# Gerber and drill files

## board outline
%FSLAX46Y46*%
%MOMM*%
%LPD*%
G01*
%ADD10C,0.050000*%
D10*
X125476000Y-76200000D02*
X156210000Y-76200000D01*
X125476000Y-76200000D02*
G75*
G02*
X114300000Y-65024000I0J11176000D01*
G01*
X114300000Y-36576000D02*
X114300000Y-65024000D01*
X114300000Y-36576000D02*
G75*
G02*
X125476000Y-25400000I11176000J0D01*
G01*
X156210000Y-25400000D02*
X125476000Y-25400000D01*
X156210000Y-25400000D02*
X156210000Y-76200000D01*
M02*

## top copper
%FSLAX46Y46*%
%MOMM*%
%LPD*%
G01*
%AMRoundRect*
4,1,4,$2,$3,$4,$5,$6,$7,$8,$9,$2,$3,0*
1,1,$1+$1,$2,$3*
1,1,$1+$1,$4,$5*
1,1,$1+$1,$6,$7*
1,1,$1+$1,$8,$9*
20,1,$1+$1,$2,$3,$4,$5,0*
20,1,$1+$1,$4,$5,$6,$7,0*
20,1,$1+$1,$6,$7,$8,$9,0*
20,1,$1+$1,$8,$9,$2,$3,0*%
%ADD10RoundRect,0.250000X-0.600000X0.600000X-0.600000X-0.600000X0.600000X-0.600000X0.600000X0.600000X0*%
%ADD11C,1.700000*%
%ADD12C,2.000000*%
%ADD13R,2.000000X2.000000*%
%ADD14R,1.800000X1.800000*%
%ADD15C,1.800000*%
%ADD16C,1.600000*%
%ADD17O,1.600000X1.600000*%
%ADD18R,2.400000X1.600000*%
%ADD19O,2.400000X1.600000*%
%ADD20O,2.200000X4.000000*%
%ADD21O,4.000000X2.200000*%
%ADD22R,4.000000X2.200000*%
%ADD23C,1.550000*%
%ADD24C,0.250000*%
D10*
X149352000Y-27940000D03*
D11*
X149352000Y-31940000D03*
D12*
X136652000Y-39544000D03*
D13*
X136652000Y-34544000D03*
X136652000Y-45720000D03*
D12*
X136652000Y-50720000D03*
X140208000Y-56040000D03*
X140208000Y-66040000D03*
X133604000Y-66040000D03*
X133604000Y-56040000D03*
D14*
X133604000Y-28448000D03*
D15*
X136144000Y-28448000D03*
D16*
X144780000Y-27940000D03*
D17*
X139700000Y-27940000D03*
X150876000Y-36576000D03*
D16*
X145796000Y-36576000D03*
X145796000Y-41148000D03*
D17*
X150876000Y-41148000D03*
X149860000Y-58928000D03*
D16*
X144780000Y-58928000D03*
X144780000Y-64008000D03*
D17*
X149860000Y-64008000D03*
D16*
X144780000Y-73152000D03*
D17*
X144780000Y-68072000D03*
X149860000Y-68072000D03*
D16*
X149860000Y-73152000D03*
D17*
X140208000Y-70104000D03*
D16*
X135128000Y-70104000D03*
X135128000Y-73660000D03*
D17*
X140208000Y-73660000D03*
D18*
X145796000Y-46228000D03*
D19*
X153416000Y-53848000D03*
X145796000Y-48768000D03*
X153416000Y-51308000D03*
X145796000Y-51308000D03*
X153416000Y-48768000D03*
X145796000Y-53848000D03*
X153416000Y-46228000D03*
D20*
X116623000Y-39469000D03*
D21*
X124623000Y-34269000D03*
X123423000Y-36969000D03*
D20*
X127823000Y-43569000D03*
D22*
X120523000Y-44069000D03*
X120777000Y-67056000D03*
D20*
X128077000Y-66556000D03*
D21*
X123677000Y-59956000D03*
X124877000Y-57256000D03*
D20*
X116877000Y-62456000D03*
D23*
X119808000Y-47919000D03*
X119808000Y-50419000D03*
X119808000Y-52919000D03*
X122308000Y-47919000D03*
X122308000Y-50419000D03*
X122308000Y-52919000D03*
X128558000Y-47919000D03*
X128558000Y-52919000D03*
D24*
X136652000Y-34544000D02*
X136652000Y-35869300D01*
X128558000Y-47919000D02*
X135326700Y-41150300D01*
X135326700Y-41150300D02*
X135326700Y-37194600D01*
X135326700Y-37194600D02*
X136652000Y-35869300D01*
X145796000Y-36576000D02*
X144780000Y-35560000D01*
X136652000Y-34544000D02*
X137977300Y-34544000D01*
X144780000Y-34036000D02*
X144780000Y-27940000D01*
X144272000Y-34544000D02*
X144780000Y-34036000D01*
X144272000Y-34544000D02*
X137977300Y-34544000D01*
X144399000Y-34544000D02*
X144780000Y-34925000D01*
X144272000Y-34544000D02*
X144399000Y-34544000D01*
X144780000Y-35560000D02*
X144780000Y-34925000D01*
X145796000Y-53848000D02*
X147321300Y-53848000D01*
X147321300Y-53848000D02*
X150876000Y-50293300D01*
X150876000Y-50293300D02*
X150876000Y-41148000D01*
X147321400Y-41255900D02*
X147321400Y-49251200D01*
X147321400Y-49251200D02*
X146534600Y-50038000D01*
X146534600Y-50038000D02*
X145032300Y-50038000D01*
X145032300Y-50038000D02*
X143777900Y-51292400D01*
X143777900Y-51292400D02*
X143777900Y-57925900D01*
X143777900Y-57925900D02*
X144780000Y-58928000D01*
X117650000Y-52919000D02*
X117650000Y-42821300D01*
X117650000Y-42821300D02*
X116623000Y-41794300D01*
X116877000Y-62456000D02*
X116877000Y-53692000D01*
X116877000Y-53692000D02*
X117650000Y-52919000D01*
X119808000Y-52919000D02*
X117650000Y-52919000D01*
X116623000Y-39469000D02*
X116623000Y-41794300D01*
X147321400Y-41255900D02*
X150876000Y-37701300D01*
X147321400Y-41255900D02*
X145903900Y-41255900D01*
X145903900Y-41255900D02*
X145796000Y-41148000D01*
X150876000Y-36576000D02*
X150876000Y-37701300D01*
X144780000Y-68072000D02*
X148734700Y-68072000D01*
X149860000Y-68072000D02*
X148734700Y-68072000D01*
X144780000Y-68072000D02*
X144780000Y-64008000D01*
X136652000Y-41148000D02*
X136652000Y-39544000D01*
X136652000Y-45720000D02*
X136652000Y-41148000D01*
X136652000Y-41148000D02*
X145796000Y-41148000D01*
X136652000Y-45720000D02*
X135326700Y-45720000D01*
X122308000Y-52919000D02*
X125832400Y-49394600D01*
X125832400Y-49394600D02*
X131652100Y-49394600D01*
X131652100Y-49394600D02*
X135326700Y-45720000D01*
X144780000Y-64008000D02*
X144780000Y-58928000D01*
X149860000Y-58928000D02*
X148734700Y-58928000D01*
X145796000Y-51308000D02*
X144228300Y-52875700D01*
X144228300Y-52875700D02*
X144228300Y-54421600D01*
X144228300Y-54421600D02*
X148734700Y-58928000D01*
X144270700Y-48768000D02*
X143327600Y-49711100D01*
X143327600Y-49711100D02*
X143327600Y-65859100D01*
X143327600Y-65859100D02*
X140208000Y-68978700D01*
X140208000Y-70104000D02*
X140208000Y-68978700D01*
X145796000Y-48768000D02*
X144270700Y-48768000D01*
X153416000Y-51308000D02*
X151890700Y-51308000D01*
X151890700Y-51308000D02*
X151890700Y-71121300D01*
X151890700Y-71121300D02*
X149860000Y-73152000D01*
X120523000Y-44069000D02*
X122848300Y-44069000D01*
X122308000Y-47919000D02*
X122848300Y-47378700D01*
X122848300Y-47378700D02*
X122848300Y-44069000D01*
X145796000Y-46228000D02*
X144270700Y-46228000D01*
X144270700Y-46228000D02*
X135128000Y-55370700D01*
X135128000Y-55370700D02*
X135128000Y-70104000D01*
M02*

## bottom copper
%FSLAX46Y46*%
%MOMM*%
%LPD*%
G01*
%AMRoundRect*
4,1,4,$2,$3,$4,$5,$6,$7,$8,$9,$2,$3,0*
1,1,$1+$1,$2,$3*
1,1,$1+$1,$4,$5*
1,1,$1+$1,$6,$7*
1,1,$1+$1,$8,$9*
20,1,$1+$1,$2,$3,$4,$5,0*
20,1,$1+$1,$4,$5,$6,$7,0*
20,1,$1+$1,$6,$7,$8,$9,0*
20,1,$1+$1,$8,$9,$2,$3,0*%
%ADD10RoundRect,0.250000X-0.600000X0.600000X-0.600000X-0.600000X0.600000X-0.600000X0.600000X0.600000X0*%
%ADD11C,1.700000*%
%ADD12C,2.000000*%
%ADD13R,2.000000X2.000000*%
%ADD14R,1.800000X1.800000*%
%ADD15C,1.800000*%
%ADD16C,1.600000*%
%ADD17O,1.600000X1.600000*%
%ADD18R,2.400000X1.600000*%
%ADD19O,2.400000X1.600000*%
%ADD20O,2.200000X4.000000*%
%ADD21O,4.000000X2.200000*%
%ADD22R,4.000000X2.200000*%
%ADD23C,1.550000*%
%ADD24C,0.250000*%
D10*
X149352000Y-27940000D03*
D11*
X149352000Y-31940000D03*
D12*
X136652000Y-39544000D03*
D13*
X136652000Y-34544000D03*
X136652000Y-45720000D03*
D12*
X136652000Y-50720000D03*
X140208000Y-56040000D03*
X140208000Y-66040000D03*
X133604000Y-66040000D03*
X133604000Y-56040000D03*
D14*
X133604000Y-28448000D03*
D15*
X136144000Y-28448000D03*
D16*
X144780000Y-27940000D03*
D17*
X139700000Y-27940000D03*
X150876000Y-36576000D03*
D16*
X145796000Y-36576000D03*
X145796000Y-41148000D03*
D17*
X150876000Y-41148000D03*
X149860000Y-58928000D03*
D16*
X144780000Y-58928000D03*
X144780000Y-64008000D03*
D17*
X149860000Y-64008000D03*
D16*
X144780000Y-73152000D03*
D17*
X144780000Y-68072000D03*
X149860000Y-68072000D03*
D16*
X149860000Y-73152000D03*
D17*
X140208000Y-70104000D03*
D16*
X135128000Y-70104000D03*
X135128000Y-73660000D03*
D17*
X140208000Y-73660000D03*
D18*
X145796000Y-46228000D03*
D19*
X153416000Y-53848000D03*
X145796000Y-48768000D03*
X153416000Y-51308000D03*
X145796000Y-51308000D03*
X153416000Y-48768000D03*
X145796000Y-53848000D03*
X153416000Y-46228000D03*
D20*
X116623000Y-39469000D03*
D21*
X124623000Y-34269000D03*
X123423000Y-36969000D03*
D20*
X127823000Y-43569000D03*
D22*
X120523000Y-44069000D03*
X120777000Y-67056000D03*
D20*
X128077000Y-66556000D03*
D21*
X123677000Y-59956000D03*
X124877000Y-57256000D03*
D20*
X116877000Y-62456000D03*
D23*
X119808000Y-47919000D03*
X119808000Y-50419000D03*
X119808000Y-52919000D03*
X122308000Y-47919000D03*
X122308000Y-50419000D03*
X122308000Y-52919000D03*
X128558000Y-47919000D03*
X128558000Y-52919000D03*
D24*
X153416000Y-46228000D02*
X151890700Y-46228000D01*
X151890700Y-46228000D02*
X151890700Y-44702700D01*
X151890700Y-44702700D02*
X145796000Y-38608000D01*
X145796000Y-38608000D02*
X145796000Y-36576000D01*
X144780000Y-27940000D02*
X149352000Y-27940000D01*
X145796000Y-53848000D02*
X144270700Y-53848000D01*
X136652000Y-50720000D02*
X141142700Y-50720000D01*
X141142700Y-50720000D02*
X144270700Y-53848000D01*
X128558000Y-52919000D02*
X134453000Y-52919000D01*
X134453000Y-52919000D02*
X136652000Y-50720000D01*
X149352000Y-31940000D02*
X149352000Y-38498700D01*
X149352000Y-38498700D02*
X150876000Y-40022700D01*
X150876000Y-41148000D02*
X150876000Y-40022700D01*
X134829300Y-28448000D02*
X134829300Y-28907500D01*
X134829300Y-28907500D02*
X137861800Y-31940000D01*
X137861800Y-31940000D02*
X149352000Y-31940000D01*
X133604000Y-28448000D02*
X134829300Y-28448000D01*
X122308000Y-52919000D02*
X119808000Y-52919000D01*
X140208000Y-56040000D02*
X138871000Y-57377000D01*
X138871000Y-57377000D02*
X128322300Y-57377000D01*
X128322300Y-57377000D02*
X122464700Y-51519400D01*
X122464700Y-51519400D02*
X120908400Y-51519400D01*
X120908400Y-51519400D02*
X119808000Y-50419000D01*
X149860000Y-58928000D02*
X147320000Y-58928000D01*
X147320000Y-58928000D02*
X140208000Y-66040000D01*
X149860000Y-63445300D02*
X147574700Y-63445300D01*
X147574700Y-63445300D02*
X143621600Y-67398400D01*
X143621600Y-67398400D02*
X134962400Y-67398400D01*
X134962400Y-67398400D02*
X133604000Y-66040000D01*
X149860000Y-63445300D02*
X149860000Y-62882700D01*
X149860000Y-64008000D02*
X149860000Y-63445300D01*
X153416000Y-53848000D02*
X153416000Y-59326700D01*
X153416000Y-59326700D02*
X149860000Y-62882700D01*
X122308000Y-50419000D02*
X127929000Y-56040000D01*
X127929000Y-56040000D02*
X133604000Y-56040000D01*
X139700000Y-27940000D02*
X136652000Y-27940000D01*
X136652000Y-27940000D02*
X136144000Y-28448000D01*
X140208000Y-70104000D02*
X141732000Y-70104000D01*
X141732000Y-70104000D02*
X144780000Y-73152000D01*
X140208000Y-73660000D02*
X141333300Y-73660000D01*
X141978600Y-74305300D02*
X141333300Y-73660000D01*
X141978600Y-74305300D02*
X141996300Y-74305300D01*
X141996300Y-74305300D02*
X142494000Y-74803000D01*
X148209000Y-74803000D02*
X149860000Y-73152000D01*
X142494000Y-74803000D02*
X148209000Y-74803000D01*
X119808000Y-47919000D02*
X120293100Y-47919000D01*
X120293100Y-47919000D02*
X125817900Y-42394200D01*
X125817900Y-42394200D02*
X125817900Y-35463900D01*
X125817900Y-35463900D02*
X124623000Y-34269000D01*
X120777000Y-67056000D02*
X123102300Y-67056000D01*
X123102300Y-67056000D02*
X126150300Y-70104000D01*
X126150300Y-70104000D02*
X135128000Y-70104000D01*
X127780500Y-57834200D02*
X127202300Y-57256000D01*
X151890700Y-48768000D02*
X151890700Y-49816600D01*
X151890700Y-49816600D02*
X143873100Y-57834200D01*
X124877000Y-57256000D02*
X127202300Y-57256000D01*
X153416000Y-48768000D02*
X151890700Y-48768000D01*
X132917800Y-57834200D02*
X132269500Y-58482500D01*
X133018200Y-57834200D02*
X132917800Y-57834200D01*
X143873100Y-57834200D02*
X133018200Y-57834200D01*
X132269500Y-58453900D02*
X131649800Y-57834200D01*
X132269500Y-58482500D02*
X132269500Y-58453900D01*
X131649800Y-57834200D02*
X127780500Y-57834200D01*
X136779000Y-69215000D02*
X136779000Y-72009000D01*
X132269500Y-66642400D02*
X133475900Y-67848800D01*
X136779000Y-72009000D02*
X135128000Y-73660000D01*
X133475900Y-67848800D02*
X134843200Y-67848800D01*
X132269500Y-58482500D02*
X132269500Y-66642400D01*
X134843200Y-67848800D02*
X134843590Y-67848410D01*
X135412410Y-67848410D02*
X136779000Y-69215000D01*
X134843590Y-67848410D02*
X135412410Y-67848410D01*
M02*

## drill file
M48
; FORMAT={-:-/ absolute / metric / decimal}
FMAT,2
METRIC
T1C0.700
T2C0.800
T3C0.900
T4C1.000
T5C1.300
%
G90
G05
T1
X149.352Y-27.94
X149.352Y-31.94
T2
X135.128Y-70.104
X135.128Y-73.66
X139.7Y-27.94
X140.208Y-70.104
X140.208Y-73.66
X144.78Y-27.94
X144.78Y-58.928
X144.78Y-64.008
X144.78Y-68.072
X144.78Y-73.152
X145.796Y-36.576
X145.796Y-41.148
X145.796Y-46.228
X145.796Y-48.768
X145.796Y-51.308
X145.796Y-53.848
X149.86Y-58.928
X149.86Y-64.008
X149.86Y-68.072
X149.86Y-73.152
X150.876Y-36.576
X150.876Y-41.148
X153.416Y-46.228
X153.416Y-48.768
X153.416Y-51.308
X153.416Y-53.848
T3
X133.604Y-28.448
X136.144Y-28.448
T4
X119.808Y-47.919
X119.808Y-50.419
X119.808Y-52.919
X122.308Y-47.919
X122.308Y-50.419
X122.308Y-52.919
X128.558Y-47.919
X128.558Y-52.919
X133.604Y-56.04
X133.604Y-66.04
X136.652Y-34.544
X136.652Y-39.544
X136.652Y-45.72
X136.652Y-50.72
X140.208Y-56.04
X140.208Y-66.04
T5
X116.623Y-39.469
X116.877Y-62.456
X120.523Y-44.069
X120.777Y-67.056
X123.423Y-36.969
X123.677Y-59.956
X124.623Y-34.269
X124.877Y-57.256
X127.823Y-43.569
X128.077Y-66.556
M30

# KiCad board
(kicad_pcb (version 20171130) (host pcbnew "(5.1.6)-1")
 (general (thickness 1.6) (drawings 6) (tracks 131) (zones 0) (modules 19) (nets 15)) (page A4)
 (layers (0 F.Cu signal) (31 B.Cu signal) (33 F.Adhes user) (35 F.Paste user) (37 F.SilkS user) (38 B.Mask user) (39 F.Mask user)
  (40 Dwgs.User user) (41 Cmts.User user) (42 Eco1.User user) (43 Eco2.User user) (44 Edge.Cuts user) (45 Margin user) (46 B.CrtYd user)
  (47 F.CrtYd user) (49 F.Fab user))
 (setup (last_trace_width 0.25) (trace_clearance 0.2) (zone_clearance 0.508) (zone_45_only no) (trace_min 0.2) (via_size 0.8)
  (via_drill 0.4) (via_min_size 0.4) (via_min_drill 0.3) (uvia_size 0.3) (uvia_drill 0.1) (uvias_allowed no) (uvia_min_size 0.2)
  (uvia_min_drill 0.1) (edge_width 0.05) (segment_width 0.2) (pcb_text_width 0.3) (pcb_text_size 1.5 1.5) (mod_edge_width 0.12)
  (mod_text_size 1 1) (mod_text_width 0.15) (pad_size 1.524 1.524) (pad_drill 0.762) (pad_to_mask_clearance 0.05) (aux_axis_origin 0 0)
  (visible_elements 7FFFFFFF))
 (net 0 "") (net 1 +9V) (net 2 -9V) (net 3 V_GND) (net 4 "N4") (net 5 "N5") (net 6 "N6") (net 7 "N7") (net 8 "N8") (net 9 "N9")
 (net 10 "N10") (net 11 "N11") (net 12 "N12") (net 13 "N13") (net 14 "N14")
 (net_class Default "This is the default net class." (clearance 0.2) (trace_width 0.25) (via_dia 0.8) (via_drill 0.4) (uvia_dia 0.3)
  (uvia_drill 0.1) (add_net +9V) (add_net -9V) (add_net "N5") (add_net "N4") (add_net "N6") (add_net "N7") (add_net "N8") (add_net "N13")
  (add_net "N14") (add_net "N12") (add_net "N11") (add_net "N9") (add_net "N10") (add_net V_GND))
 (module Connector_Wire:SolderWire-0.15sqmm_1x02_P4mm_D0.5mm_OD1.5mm (layer F.Cu) (at 149.352 27.94 270)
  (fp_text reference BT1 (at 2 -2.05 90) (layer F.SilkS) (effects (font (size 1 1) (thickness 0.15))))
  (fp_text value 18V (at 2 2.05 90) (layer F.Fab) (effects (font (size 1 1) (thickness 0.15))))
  (pad 1 thru_hole roundrect (at 0 0 270) (size 1.7 1.7) (drill 0.7) (layers *.Cu *.Mask) (roundrect_rratio 0.147059) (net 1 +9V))
  (pad 2 thru_hole circle (at 4 0 270) (size 1.7 1.7) (drill 0.7) (layers *.Cu *.Mask) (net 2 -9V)))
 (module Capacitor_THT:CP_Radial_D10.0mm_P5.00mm (layer F.Cu) (at 136.652 34.544 270)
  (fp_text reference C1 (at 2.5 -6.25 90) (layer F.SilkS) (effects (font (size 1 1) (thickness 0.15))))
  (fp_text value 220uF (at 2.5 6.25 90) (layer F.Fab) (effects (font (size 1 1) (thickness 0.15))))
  (pad 2 thru_hole circle (at 5 0 270) (size 2 2) (drill 1) (layers *.Cu *.Mask) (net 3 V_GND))
  (pad 1 thru_hole rect (at 0 0 270) (size 2 2) (drill 1) (layers *.Cu *.Mask) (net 1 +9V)))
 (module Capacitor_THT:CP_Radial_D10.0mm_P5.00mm (layer F.Cu) (at 136.652 45.72 270)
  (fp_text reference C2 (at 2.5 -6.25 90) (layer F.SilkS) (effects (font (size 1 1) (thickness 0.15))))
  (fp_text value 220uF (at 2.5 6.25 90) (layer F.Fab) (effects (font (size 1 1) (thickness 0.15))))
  (pad 1 thru_hole rect (at 0 0 270) (size 2 2) (drill 1) (layers *.Cu *.Mask) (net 3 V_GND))
  (pad 2 thru_hole circle (at 5 0 270) (size 2 2) (drill 1) (layers *.Cu *.Mask) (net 2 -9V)))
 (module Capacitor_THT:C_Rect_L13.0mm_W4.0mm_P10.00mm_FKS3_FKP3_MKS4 (layer F.Cu) (at 140.208 66.04 90)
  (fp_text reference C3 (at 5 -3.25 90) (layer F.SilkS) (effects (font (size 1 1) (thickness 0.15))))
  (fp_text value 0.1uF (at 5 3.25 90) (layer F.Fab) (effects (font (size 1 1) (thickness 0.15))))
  (pad 2 thru_hole circle (at 10 0 90) (size 2 2) (drill 1) (layers *.Cu *.Mask) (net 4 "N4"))
  (pad 1 thru_hole circle (at 0 0 90) (size 2 2) (drill 1) (layers *.Cu *.Mask) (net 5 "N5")))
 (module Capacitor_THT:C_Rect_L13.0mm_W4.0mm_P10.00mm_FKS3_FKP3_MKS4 (layer F.Cu) (at 133.604 66.04 90)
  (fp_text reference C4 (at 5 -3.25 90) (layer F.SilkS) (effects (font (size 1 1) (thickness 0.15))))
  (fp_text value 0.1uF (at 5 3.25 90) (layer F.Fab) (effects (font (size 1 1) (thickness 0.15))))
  (pad 1 thru_hole circle (at 0 0 90) (size 2 2) (drill 1) (layers *.Cu *.Mask) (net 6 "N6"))
  (pad 2 thru_hole circle (at 10 0 90) (size 2 2) (drill 1) (layers *.Cu *.Mask) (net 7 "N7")))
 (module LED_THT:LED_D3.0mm (layer F.Cu) (at 133.604 28.448)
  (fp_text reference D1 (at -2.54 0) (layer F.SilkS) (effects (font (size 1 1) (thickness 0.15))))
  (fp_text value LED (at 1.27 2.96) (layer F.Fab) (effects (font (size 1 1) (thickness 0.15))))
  (pad 1 thru_hole rect (at 0 0) (size 1.8 1.8) (drill 0.9) (layers *.Cu *.Mask) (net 2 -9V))
  (pad 2 thru_hole circle (at 2.54 0) (size 1.8 1.8) (drill 0.9) (layers *.Cu *.Mask) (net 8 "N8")))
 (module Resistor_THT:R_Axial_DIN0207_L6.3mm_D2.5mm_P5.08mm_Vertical (layer F.Cu) (at 144.78 27.94 180)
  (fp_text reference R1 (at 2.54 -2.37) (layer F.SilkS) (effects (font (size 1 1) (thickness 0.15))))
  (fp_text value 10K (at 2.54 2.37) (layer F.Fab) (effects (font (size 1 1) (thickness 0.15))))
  (pad 1 thru_hole circle (at 0 0 180) (size 1.6 1.6) (drill 0.8) (layers *.Cu *.Mask) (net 1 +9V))
  (pad 2 thru_hole oval (at 5.08 0 180) (size 1.6 1.6) (drill 0.8) (layers *.Cu *.Mask) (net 8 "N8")))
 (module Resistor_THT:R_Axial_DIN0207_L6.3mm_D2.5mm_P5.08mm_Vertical (layer F.Cu) (at 145.796 36.576)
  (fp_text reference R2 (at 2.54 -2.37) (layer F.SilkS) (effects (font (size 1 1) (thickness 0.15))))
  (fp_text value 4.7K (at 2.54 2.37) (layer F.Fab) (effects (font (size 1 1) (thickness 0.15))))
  (pad 2 thru_hole oval (at 5.08 0) (size 1.6 1.6) (drill 0.8) (layers *.Cu *.Mask) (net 3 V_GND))
  (pad 1 thru_hole circle (at 0 0) (size 1.6 1.6) (drill 0.8) (layers *.Cu *.Mask) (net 1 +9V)))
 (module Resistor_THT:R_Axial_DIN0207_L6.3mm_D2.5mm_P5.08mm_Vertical (layer F.Cu) (at 145.796 41.148)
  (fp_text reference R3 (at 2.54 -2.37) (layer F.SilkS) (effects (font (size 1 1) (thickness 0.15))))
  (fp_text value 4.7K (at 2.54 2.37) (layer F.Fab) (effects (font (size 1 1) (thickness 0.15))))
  (pad 1 thru_hole circle (at 0 0) (size 1.6 1.6) (drill 0.8) (layers *.Cu *.Mask) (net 3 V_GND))
  (pad 2 thru_hole oval (at 5.08 0) (size 1.6 1.6) (drill 0.8) (layers *.Cu *.Mask) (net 2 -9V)))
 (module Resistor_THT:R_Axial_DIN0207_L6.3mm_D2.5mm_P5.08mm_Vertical (layer F.Cu) (at 144.78 58.928)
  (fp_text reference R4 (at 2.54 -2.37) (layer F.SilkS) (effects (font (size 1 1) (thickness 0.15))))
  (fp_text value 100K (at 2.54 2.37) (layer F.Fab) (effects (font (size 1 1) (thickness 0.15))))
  (pad 2 thru_hole oval (at 5.08 0) (size 1.6 1.6) (drill 0.8) (layers *.Cu *.Mask) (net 5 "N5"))
  (pad 1 thru_hole circle (at 0 0) (size 1.6 1.6) (drill 0.8) (layers *.Cu *.Mask) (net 3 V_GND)))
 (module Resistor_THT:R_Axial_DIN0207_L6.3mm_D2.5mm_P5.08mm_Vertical (layer F.Cu) (at 144.78 64.008)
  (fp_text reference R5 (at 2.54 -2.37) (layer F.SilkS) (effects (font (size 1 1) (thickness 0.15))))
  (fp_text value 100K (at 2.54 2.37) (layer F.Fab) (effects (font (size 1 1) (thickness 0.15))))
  (pad 1 thru_hole circle (at 0 0) (size 1.6 1.6) (drill 0.8) (layers *.Cu *.Mask) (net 3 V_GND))
  (pad 2 thru_hole oval (at 5.08 0) (size 1.6 1.6) (drill 0.8) (layers *.Cu *.Mask) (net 6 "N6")))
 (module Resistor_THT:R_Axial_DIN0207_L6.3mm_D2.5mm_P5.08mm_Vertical (layer F.Cu) (at 144.78 73.152 90)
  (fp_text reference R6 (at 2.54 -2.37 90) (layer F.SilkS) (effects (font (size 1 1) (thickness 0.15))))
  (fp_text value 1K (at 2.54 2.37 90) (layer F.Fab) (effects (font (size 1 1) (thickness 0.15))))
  (pad 1 thru_hole circle (at 0 0 90) (size 1.6 1.6) (drill 0.8) (layers *.Cu *.Mask) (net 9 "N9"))
  (pad 2 thru_hole oval (at 5.08 0 90) (size 1.6 1.6) (drill 0.8) (layers *.Cu *.Mask) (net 3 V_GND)))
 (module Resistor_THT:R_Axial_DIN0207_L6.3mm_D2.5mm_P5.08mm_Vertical (layer F.Cu) (at 149.86 73.152 90)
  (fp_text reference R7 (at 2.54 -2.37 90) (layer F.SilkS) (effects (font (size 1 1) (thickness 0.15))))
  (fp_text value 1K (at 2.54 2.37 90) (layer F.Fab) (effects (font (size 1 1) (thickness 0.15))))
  (pad 2 thru_hole oval (at 5.08 0 90) (size 1.6 1.6) (drill 0.8) (layers *.Cu *.Mask) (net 3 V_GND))
  (pad 1 thru_hole circle (at 0 0 90) (size 1.6 1.6) (drill 0.8) (layers *.Cu *.Mask) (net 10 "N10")))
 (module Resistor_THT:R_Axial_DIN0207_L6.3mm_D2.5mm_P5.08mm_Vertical (layer F.Cu) (at 135.128 70.104)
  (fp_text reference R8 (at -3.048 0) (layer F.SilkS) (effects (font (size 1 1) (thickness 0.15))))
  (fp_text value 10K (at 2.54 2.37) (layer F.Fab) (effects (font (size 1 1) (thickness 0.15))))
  (pad 2 thru_hole oval (at 5.08 0) (size 1.6 1.6) (drill 0.8) (layers *.Cu *.Mask) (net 9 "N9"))
  (pad 1 thru_hole circle (at 0 0) (size 1.6 1.6) (drill 0.8) (layers *.Cu *.Mask) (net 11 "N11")))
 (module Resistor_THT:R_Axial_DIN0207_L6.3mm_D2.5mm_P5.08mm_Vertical (layer F.Cu) (at 135.128 73.66)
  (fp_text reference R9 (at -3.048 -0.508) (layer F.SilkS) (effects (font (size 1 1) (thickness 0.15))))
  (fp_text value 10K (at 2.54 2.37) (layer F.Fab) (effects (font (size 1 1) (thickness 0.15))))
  (pad 1 thru_hole circle (at 0 0) (size 1.6 1.6) (drill 0.8) (layers *.Cu *.Mask) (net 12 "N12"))
  (pad 2 thru_hole oval (at 5.08 0) (size 1.6 1.6) (drill 0.8) (layers *.Cu *.Mask) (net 10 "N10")))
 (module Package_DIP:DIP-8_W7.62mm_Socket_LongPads (layer F.Cu) (at 145.796 46.228)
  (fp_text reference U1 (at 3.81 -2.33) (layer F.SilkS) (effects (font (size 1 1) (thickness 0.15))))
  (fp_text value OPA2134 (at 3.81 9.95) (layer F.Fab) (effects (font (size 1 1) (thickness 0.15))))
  (pad 1 thru_hole rect (at 0 0) (size 2.4 1.6) (drill 0.8) (layers *.Cu *.Mask) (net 11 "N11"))
  (pad 5 thru_hole oval (at 7.62 7.62) (size 2.4 1.6) (drill 0.8) (layers *.Cu *.Mask) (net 6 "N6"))
  (pad 2 thru_hole oval (at 0 2.54) (size 2.4 1.6) (drill 0.8) (layers *.Cu *.Mask) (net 9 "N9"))
  (pad 6 thru_hole oval (at 7.62 5.08) (size 2.4 1.6) (drill 0.8) (layers *.Cu *.Mask) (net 10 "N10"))
  (pad 3 thru_hole oval (at 0 5.08) (size 2.4 1.6) (drill 0.8) (layers *.Cu *.Mask) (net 5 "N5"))
  (pad 7 thru_hole oval (at 7.62 2.54) (size 2.4 1.6) (drill 0.8) (layers *.Cu *.Mask) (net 12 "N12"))
  (pad 4 thru_hole oval (at 0 7.62) (size 2.4 1.6) (drill 0.8) (layers *.Cu *.Mask) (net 2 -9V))
  (pad 8 thru_hole oval (at 7.62 0) (size 2.4 1.6) (drill 0.8) (layers *.Cu *.Mask) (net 1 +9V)))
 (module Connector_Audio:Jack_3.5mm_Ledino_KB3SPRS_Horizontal (layer F.Cu) (at 120.523 44.069)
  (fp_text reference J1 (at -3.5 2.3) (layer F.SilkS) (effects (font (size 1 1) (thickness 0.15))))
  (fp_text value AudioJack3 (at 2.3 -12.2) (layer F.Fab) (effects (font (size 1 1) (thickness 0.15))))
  (pad S thru_hole oval (at -3.9 -4.6) (size 2.2 4) (drill 1.3) (layers *.Cu *.Mask) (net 3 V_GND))
  (pad R thru_hole oval (at 4.1 -9.8) (size 4 2.2) (drill 1.3) (layers *.Cu *.Mask) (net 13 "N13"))
  (pad RN thru_hole oval (at 2.9 -7.1) (size 4 2.2) (drill 1.3) (layers *.Cu *.Mask))
  (pad TN thru_hole oval (at 7.3 -0.5 90) (size 4 2.2) (drill 1.3) (layers *.Cu *.Mask))
  (pad T thru_hole rect (at 0 0) (size 4 2.2) (drill 1.3) (layers *.Cu *.Mask) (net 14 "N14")))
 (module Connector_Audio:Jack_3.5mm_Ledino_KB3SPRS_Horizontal (layer F.Cu) (at 120.777 67.056)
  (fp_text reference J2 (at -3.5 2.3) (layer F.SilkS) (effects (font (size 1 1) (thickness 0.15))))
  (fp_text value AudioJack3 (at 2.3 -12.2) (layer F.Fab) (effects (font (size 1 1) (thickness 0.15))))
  (pad T thru_hole rect (at 0 0) (size 4 2.2) (drill 1.3) (layers *.Cu *.Mask) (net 11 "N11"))
  (pad TN thru_hole oval (at 7.3 -0.5 90) (size 4 2.2) (drill 1.3) (layers *.Cu *.Mask))
  (pad RN thru_hole oval (at 2.9 -7.1) (size 4 2.2) (drill 1.3) (layers *.Cu *.Mask))
  (pad R thru_hole oval (at 4.1 -9.8) (size 4 2.2) (drill 1.3) (layers *.Cu *.Mask) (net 12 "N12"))
  (pad S thru_hole oval (at -3.9 -4.6) (size 2.2 4) (drill 1.3) (layers *.Cu *.Mask) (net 3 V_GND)))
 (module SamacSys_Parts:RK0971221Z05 (layer F.Cu) (at 114.808 50.419 180)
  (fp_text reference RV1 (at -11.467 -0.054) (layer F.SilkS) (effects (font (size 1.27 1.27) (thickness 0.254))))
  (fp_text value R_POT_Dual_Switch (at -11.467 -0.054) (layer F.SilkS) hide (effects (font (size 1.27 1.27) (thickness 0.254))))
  (pad 1 thru_hole circle (at -5 2.5 180) (size 1.55 1.55) (drill 1) (layers *.Cu *.Mask) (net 13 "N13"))
  (pad 2 thru_hole circle (at -5 0 180) (size 1.55 1.55) (drill 1) (layers *.Cu *.Mask) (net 4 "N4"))
  (pad 3 thru_hole circle (at -5 -2.5 180) (size 1.55 1.55) (drill 1) (layers *.Cu *.Mask) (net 3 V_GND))
  (pad 4 thru_hole circle (at -7.5 2.5 180) (size 1.55 1.55) (drill 1) (layers *.Cu *.Mask) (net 14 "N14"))
  (pad 5 thru_hole circle (at -7.5 0 180) (size 1.55 1.55) (drill 1) (layers *.Cu *.Mask) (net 7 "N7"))
  (pad 6 thru_hole circle (at -7.5 -2.5 180) (size 1.55 1.55) (drill 1) (layers *.Cu *.Mask) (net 3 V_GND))
  (pad 7 thru_hole circle (at -13.75 2.5 180) (size 1.55 1.55) (drill 1) (layers *.Cu *.Mask) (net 1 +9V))
  (pad 8 thru_hole circle (at -13.75 -2.5 180) (size 1.55 1.55) (drill 1) (layers *.Cu *.Mask) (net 2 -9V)))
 (gr_line (start 125.476 76.2) (end 156.21 76.2) (layer Edge.Cuts) (width 0.05))
 (gr_arc (start 125.476 65.024) (end 114.3 65.024) (angle -90) (layer Edge.Cuts) (width 0.05))
 (gr_line (start 114.3 36.576) (end 114.3 65.024) (layer Edge.Cuts) (width 0.05))
 (gr_arc (start 125.476 36.576) (end 125.476 25.4) (angle -90) (layer Edge.Cuts) (width 0.05))
 (gr_line (start 156.21 25.4) (end 125.476 25.4) (layer Edge.Cuts) (width 0.05))
 (gr_line (start 156.21 25.4) (end 156.21 76.2) (layer Edge.Cuts) (width 0.05))
 (segment (start 153.416 46.228) (end 151.8907 46.228) (width 0.25) (layer B.Cu) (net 1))
 (segment (start 151.8907 46.228) (end 151.8907 44.7027) (width 0.25) (layer B.Cu) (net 1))
 (segment (start 151.8907 44.7027) (end 145.796 38.608) (width 0.25) (layer B.Cu) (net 1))
 (segment (start 145.796 38.608) (end 145.796 36.576) (width 0.25) (layer B.Cu) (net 1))
 (segment (start 136.652 34.544) (end 136.652 35.8693) (width 0.25) (layer F.Cu) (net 1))
 (segment (start 128.558 47.919) (end 135.3267 41.1503) (width 0.25) (layer F.Cu) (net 1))
 (segment (start 135.3267 41.1503) (end 135.3267 37.1946) (width 0.25) (layer F.Cu) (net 1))
 (segment (start 135.3267 37.1946) (end 136.652 35.8693) (width 0.25) (layer F.Cu) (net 1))
 (segment (start 145.796 36.576) (end 144.78 35.56) (width 0.25) (layer F.Cu) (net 1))
 (segment (start 136.652 34.544) (end 137.9773 34.544) (width 0.25) (layer F.Cu) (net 1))
 (segment (start 144.78 27.94) (end 149.352 27.94) (width 0.25) (layer B.Cu) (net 1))
 (segment (start 144.78 34.036) (end 144.78 27.94) (width 0.25) (layer F.Cu) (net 1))
 (segment (start 144.272 34.544) (end 144.78 34.036) (width 0.25) (layer F.Cu) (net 1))
 (segment (start 144.272 34.544) (end 137.9773 34.544) (width 0.25) (layer F.Cu) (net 1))
 (segment (start 144.399 34.544) (end 144.78 34.925) (width 0.25) (layer F.Cu) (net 1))
 (segment (start 144.272 34.544) (end 144.399 34.544) (width 0.25) (layer F.Cu) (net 1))
 (segment (start 144.78 35.56) (end 144.78 34.925) (width 0.25) (layer F.Cu) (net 1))
 (segment (start 145.796 53.848) (end 147.3213 53.848) (width 0.25) (layer F.Cu) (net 2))
 (segment (start 147.3213 53.848) (end 150.876 50.2933) (width 0.25) (layer F.Cu) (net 2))
 (segment (start 150.876 50.2933) (end 150.876 41.148) (width 0.25) (layer F.Cu) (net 2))
 (segment (start 145.796 53.848) (end 144.2707 53.848) (width 0.25) (layer B.Cu) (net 2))
 (segment (start 136.652 50.72) (end 141.1427 50.72) (width 0.25) (layer B.Cu) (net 2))
 (segment (start 141.1427 50.72) (end 144.2707 53.848) (width 0.25) (layer B.Cu) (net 2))
 (segment (start 128.558 52.919) (end 134.453 52.919) (width 0.25) (layer B.Cu) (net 2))
 (segment (start 134.453 52.919) (end 136.652 50.72) (width 0.25) (layer B.Cu) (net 2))
 (segment (start 149.352 31.94) (end 149.352 38.4987) (width 0.25) (layer B.Cu) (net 2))
 (segment (start 149.352 38.4987) (end 150.876 40.0227) (width 0.25) (layer B.Cu) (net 2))
 (segment (start 150.876 41.148) (end 150.876 40.0227) (width 0.25) (layer B.Cu) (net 2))
 (segment (start 134.8293 28.448) (end 134.8293 28.9075) (width 0.25) (layer B.Cu) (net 2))
 (segment (start 134.8293 28.9075) (end 137.8618 31.94) (width 0.25) (layer B.Cu) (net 2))
 (segment (start 137.8618 31.94) (end 149.352 31.94) (width 0.25) (layer B.Cu) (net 2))
 (segment (start 133.604 28.448) (end 134.8293 28.448) (width 0.25) (layer B.Cu) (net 2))
 (segment (start 147.3214 41.2559) (end 147.3214 49.2512) (width 0.25) (layer F.Cu) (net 3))
 (segment (start 147.3214 49.2512) (end 146.5346 50.038) (width 0.25) (layer F.Cu) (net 3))
 (segment (start 146.5346 50.038) (end 145.0323 50.038) (width 0.25) (layer F.Cu) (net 3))
 (segment (start 145.0323 50.038) (end 143.7779 51.2924) (width 0.25) (layer F.Cu) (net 3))
 (segment (start 143.7779 51.2924) (end 143.7779 57.9259) (width 0.25) (layer F.Cu) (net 3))
 (segment (start 143.7779 57.9259) (end 144.78 58.928) (width 0.25) (layer F.Cu) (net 3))
 (segment (start 117.65 52.919) (end 117.65 42.8213) (width 0.25) (layer F.Cu) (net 3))
 (segment (start 117.65 42.8213) (end 116.623 41.7943) (width 0.25) (layer F.Cu) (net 3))
 (segment (start 116.877 62.456) (end 116.877 53.692) (width 0.25) (layer F.Cu) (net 3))
 (segment (start 116.877 53.692) (end 117.65 52.919) (width 0.25) (layer F.Cu) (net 3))
 (segment (start 119.808 52.919) (end 117.65 52.919) (width 0.25) (layer F.Cu) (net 3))
 (segment (start 116.623 39.469) (end 116.623 41.7943) (width 0.25) (layer F.Cu) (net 3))
 (segment (start 147.3214 41.2559) (end 150.876 37.7013) (width 0.25) (layer F.Cu) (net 3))
 (segment (start 147.3214 41.2559) (end 145.9039 41.2559) (width 0.25) (layer F.Cu) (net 3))
 (segment (start 145.9039 41.2559) (end 145.796 41.148) (width 0.25) (layer F.Cu) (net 3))
 (segment (start 150.876 36.576) (end 150.876 37.7013) (width 0.25) (layer F.Cu) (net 3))
 (segment (start 144.78 68.072) (end 148.7347 68.072) (width 0.25) (layer F.Cu) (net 3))
 (segment (start 149.86 68.072) (end 148.7347 68.072) (width 0.25) (layer F.Cu) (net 3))
 (segment (start 144.78 68.072) (end 144.78 64.008) (width 0.25) (layer F.Cu) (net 3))
 (segment (start 136.652 41.148) (end 136.652 39.544) (width 0.25) (layer F.Cu) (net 3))
 (segment (start 136.652 45.72) (end 136.652 41.148) (width 0.25) (layer F.Cu) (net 3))
 (segment (start 136.652 41.148) (end 145.796 41.148) (width 0.25) (layer F.Cu) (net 3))
 (segment (start 136.652 45.72) (end 135.3267 45.72) (width 0.25) (layer F.Cu) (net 3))
 (segment (start 122.308 52.919) (end 125.8324 49.3946) (width 0.25) (layer F.Cu) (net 3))
 (segment (start 125.8324 49.3946) (end 131.6521 49.3946) (width 0.25) (layer F.Cu) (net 3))
 (segment (start 131.6521 49.3946) (end 135.3267 45.72) (width 0.25) (layer F.Cu) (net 3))
 (segment (start 144.78 64.008) (end 144.78 58.928) (width 0.25) (layer F.Cu) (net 3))
 (segment (start 122.308 52.919) (end 119.808 52.919) (width 0.25) (layer B.Cu) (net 3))
 (segment (start 140.208 56.04) (end 138.871 57.377) (width 0.25) (layer B.Cu) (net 4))
 (segment (start 138.871 57.377) (end 128.3223 57.377) (width 0.25) (layer B.Cu) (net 4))
 (segment (start 128.3223 57.377) (end 122.4647 51.5194) (width 0.25) (layer B.Cu) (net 4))
 (segment (start 122.4647 51.5194) (end 120.9084 51.5194) (width 0.25) (layer B.Cu) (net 4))
 (segment (start 120.9084 51.5194) (end 119.808 50.419) (width 0.25) (layer B.Cu) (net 4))
 (segment (start 149.86 58.928) (end 148.7347 58.928) (width 0.25) (layer F.Cu) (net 5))
 (segment (start 145.796 51.308) (end 144.2283 52.8757) (width 0.25) (layer F.Cu) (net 5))
 (segment (start 144.2283 52.8757) (end 144.2283 54.4216) (width 0.25) (layer F.Cu) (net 5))
 (segment (start 144.2283 54.4216) (end 148.7347 58.928) (width 0.25) (layer F.Cu) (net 5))
 (segment (start 149.86 58.928) (end 147.32 58.928) (width 0.25) (layer B.Cu) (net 5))
 (segment (start 147.32 58.928) (end 140.208 66.04) (width 0.25) (layer B.Cu) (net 5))
 (segment (start 149.86 63.4453) (end 147.5747 63.4453) (width 0.25) (layer B.Cu) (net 6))
 (segment (start 147.5747 63.4453) (end 143.6216 67.3984) (width 0.25) (layer B.Cu) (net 6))
 (segment (start 143.6216 67.3984) (end 134.9624 67.3984) (width 0.25) (layer B.Cu) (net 6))
 (segment (start 134.9624 67.3984) (end 133.604 66.04) (width 0.25) (layer B.Cu) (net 6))
 (segment (start 149.86 63.4453) (end 149.86 62.8827) (width 0.25) (layer B.Cu) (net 6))
 (segment (start 149.86 64.008) (end 149.86 63.4453) (width 0.25) (layer B.Cu) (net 6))
 (segment (start 153.416 53.848) (end 153.416 59.3267) (width 0.25) (layer B.Cu) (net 6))
 (segment (start 153.416 59.3267) (end 149.86 62.8827) (width 0.25) (layer B.Cu) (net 6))
 (segment (start 122.308 50.419) (end 127.929 56.04) (width 0.25) (layer B.Cu) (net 7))
 (segment (start 127.929 56.04) (end 133.604 56.04) (width 0.25) (layer B.Cu) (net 7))
 (segment (start 139.7 27.94) (end 136.652 27.94) (width 0.25) (layer B.Cu) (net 8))
 (segment (start 136.652 27.94) (end 136.144 28.448) (width 0.25) (layer B.Cu) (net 8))
 (segment (start 144.2707 48.768) (end 143.3276 49.7111) (width 0.25) (layer F.Cu) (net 9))
 (segment (start 143.3276 49.7111) (end 143.3276 65.8591) (width 0.25) (layer F.Cu) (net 9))
 (segment (start 143.3276 65.8591) (end 140.208 68.9787) (width 0.25) (layer F.Cu) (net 9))
 (segment (start 140.208 70.104) (end 141.732 70.104) (width 0.25) (layer B.Cu) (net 9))
 (segment (start 141.732 70.104) (end 144.78 73.152) (width 0.25) (layer B.Cu) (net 9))
 (segment (start 140.208 70.104) (end 140.208 68.9787) (width 0.25) (layer F.Cu) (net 9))
 (segment (start 145.796 48.768) (end 144.2707 48.768) (width 0.25) (layer F.Cu) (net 9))
 (segment (start 153.416 51.308) (end 151.8907 51.308) (width 0.25) (layer F.Cu) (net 10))
 (segment (start 151.8907 51.308) (end 151.8907 71.1213) (width 0.25) (layer F.Cu) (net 10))
 (segment (start 151.8907 71.1213) (end 149.86 73.152) (width 0.25) (layer F.Cu) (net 10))
 (segment (start 140.208 73.66) (end 141.3333 73.66) (width 0.25) (layer B.Cu) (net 10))
 (segment (start 141.9786 74.3053) (end 141.3333 73.66) (width 0.25) (layer B.Cu) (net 10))
 (segment (start 141.9786 74.3053) (end 141.9963 74.3053) (width 0.25) (layer B.Cu) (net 10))
 (segment (start 141.9963 74.3053) (end 142.494 74.803) (width 0.25) (layer B.Cu) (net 10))
 (segment (start 148.209 74.803) (end 149.86 73.152) (width 0.25) (layer B.Cu) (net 10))
 (segment (start 142.494 74.803) (end 148.209 74.803) (width 0.25) (layer B.Cu) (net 10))
 (segment (start 119.808 47.919) (end 120.2931 47.919) (width 0.25) (layer B.Cu) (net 13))
 (segment (start 120.2931 47.919) (end 125.8179 42.3942) (width 0.25) (layer B.Cu) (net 13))
 (segment (start 125.8179 42.3942) (end 125.8179 35.4639) (width 0.25) (layer B.Cu) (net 13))
 (segment (start 125.8179 35.4639) (end 124.623 34.269) (width 0.25) (layer B.Cu) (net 13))
 (segment (start 120.523 44.069) (end 122.8483 44.069) (width 0.25) (layer F.Cu) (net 14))
 (segment (start 122.308 47.919) (end 122.8483 47.3787) (width 0.25) (layer F.Cu) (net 14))
 (segment (start 122.8483 47.3787) (end 122.8483 44.069) (width 0.25) (layer F.Cu) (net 14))
 (segment (start 120.777 67.056) (end 123.1023 67.056) (width 0.25) (layer B.Cu) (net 11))
 (segment (start 123.1023 67.056) (end 126.1503 70.104) (width 0.25) (layer B.Cu) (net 11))
 (segment (start 126.1503 70.104) (end 135.128 70.104) (width 0.25) (layer B.Cu) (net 11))
 (segment (start 145.796 46.228) (end 144.2707 46.228) (width 0.25) (layer F.Cu) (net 11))
 (segment (start 144.2707 46.228) (end 135.128 55.3707) (width 0.25) (layer F.Cu) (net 11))
 (segment (start 135.128 55.3707) (end 135.128 70.104) (width 0.25) (layer F.Cu) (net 11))
 (segment (start 127.7805 57.8342) (end 127.2023 57.256) (width 0.25) (layer B.Cu) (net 12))
 (segment (start 151.8907 48.768) (end 151.8907 49.8166) (width 0.25) (layer B.Cu) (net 12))
 (segment (start 151.8907 49.8166) (end 143.8731 57.8342) (width 0.25) (layer B.Cu) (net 12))
 (segment (start 124.877 57.256) (end 127.2023 57.256) (width 0.25) (layer B.Cu) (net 12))
 (segment (start 153.416 48.768) (end 151.8907 48.768) (width 0.25) (layer B.Cu) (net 12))
 (segment (start 132.9178 57.8342) (end 132.2695 58.4825) (width 0.25) (layer B.Cu) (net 12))
 (segment (start 133.0182 57.8342) (end 132.9178 57.8342) (width 0.25) (layer B.Cu) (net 12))
 (segment (start 143.8731 57.8342) (end 133.0182 57.8342) (width 0.25) (layer B.Cu) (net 12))
 (segment (start 132.2695 58.4539) (end 131.6498 57.8342) (width 0.25) (layer B.Cu) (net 12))
 (segment (start 132.2695 58.4825) (end 132.2695 58.4539) (width 0.25) (layer B.Cu) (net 12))
 (segment (start 131.6498 57.8342) (end 127.7805 57.8342) (width 0.25) (layer B.Cu) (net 12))
 (segment (start 136.779 69.215) (end 136.779 72.009) (width 0.25) (layer B.Cu) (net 12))
 (segment (start 132.2695 66.6424) (end 133.4759 67.8488) (width 0.25) (layer B.Cu) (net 12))
 (segment (start 136.779 72.009) (end 135.128 73.66) (width 0.25) (layer B.Cu) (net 12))
 (segment (start 133.4759 67.8488) (end 134.8432 67.8488) (width 0.25) (layer B.Cu) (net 12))
 (segment (start 132.2695 58.4825) (end 132.2695 66.6424) (width 0.25) (layer B.Cu) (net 12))
 (segment (start 134.8432 67.8488) (end 134.84359 67.84841) (width 0.25) (layer B.Cu) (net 12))
 (segment (start 135.41241 67.84841) (end 136.779 69.215) (width 0.25) (layer B.Cu) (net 12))
 (segment (start 134.84359 67.84841) (end 135.41241 67.84841) (width 0.25) (layer B.Cu) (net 12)))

